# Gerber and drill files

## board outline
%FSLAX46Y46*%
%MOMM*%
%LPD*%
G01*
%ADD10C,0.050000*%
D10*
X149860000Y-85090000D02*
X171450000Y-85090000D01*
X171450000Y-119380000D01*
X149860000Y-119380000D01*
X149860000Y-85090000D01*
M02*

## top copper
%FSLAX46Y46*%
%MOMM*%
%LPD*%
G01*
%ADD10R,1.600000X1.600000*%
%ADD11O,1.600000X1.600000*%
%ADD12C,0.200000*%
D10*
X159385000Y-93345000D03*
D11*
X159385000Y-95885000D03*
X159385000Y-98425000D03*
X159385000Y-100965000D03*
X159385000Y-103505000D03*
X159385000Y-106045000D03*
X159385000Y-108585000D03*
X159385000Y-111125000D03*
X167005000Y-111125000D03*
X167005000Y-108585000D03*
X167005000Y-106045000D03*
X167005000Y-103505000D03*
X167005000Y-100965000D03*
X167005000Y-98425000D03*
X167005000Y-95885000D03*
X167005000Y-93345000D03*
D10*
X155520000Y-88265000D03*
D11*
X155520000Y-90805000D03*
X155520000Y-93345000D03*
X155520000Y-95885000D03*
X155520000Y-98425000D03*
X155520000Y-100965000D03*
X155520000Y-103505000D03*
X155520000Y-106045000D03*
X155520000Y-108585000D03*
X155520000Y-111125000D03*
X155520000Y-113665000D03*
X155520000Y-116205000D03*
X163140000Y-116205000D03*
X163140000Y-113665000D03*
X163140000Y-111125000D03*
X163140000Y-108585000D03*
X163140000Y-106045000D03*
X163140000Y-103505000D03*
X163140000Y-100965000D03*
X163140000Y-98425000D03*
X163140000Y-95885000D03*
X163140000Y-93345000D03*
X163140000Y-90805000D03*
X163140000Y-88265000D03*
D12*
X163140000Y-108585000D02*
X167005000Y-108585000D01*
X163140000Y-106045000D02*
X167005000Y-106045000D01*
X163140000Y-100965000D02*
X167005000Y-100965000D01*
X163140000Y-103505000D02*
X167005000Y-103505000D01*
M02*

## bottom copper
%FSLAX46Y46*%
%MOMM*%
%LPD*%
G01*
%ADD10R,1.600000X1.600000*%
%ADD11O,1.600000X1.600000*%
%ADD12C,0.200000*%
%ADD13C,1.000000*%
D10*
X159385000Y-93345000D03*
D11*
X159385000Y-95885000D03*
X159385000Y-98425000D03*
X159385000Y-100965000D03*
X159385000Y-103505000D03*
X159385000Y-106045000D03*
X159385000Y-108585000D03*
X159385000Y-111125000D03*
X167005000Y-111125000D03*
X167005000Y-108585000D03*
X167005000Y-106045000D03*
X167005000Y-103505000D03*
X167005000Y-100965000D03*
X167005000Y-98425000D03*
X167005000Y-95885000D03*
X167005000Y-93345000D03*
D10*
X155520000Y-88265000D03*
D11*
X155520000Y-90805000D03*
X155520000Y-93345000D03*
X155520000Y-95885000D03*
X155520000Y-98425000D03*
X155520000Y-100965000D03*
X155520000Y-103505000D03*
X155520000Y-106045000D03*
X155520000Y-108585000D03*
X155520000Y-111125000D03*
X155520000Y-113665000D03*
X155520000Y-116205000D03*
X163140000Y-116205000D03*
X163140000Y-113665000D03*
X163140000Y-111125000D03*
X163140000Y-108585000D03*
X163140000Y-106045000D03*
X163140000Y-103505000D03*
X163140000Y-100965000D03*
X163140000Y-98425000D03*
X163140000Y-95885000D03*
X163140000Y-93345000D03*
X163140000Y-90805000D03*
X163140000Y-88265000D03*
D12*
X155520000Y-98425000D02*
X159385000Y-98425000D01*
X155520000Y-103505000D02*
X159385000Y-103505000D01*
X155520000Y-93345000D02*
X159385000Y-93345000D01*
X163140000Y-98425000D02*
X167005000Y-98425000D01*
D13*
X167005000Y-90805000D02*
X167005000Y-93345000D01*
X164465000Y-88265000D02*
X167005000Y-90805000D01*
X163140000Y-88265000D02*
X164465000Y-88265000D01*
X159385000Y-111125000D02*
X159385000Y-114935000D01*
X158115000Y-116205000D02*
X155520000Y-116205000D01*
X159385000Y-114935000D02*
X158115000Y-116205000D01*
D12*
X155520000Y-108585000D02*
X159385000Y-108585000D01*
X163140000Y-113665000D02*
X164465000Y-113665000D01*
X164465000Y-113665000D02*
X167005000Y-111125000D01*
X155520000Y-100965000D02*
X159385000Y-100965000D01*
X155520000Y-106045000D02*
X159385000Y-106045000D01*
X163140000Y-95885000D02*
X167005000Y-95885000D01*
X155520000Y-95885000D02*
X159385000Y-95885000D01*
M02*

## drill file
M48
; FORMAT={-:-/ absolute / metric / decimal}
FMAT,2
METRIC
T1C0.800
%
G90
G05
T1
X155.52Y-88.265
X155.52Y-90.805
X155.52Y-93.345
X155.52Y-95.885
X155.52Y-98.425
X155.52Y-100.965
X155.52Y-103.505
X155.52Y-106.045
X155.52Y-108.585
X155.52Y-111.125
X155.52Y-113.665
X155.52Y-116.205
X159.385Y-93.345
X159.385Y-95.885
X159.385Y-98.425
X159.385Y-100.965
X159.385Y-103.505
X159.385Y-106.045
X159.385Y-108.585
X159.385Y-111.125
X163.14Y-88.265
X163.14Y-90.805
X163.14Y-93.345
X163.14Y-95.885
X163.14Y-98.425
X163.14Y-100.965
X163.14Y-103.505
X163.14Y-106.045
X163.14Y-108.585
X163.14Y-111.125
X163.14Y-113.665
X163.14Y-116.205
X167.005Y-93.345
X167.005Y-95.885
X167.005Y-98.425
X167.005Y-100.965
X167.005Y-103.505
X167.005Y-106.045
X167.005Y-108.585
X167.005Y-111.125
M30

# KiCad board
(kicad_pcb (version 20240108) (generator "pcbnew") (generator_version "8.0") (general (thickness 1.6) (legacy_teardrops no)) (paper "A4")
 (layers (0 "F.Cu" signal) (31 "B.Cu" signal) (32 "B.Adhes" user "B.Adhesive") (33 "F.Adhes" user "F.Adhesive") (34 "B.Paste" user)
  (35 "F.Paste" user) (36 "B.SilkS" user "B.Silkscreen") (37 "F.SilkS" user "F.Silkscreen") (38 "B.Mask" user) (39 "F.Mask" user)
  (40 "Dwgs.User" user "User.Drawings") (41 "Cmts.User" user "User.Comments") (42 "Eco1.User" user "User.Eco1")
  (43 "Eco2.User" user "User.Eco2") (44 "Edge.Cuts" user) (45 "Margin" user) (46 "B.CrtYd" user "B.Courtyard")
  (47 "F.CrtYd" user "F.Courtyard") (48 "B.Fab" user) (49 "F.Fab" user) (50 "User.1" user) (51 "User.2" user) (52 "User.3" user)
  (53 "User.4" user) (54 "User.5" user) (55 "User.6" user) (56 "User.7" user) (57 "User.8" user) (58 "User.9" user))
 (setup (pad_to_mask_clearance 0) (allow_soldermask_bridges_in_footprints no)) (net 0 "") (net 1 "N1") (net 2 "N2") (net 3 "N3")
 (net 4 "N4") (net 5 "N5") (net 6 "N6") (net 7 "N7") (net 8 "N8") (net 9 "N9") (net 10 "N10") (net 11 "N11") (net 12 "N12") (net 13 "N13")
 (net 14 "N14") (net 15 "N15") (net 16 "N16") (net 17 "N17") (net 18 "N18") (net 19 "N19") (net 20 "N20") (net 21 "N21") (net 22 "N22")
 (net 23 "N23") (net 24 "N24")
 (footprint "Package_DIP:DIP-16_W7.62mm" (layer "F.Cu") (at 159.385 93.345)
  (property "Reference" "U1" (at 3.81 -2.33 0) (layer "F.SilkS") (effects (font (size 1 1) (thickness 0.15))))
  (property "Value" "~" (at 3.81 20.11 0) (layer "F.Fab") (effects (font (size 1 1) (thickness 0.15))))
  (pad "1" thru_hole rect (at 0 0) (size 1.6 1.6) (drill 0.8) (layers "*.Cu" "*.Mask") (remove_unused_layers no) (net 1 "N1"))
  (pad "2" thru_hole oval (at 0 2.54) (size 1.6 1.6) (drill 0.8) (layers "*.Cu" "*.Mask") (remove_unused_layers no) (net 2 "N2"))
  (pad "3" thru_hole oval (at 0 5.08) (size 1.6 1.6) (drill 0.8) (layers "*.Cu" "*.Mask") (remove_unused_layers no) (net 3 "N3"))
  (pad "4" thru_hole oval (at 0 7.62) (size 1.6 1.6) (drill 0.8) (layers "*.Cu" "*.Mask") (remove_unused_layers no) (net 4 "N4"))
  (pad "5" thru_hole oval (at 0 10.16) (size 1.6 1.6) (drill 0.8) (layers "*.Cu" "*.Mask") (remove_unused_layers no) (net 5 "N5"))
  (pad "6" thru_hole oval (at 0 12.7) (size 1.6 1.6) (drill 0.8) (layers "*.Cu" "*.Mask") (remove_unused_layers no) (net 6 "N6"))
  (pad "7" thru_hole oval (at 0 15.24) (size 1.6 1.6) (drill 0.8) (layers "*.Cu" "*.Mask") (remove_unused_layers no) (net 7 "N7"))
  (pad "8" thru_hole oval (at 0 17.78) (size 1.6 1.6) (drill 0.8) (layers "*.Cu" "*.Mask") (remove_unused_layers no) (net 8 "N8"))
  (pad "9" thru_hole oval (at 7.62 17.78) (size 1.6 1.6) (drill 0.8) (layers "*.Cu" "*.Mask") (remove_unused_layers no) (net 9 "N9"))
  (pad "10" thru_hole oval (at 7.62 15.24) (size 1.6 1.6) (drill 0.8) (layers "*.Cu" "*.Mask") (remove_unused_layers no) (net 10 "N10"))
  (pad "11" thru_hole oval (at 7.62 12.7) (size 1.6 1.6) (drill 0.8) (layers "*.Cu" "*.Mask") (remove_unused_layers no) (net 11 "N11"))
  (pad "12" thru_hole oval (at 7.62 10.16) (size 1.6 1.6) (drill 0.8) (layers "*.Cu" "*.Mask") (remove_unused_layers no) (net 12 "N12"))
  (pad "13" thru_hole oval (at 7.62 7.62) (size 1.6 1.6) (drill 0.8) (layers "*.Cu" "*.Mask") (remove_unused_layers no) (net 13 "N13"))
  (pad "14" thru_hole oval (at 7.62 5.08) (size 1.6 1.6) (drill 0.8) (layers "*.Cu" "*.Mask") (remove_unused_layers no) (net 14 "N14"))
  (pad "15" thru_hole oval (at 7.62 2.54) (size 1.6 1.6) (drill 0.8) (layers "*.Cu" "*.Mask") (remove_unused_layers no) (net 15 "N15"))
  (pad "16" thru_hole oval (at 7.62 0) (size 1.6 1.6) (drill 0.8) (layers "*.Cu" "*.Mask") (remove_unused_layers no) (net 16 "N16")))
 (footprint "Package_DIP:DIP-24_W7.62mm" (layer "F.Cu") (at 155.52 88.265)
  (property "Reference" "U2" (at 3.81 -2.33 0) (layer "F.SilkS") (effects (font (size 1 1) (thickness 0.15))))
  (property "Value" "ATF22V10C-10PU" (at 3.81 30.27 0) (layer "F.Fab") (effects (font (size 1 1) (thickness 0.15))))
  (pad "1" thru_hole rect (at 0 0) (size 1.6 1.6) (drill 0.8) (layers "*.Cu" "*.Mask") (remove_unused_layers no) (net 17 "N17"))
  (pad "2" thru_hole oval (at 0 2.54) (size 1.6 1.6) (drill 0.8) (layers "*.Cu" "*.Mask") (remove_unused_layers no) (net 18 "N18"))
  (pad "3" thru_hole oval (at 0 5.08) (size 1.6 1.6) (drill 0.8) (layers "*.Cu" "*.Mask") (remove_unused_layers no) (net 1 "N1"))
  (pad "4" thru_hole oval (at 0 7.62) (size 1.6 1.6) (drill 0.8) (layers "*.Cu" "*.Mask") (remove_unused_layers no) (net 2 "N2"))
  (pad "5" thru_hole oval (at 0 10.16) (size 1.6 1.6) (drill 0.8) (layers "*.Cu" "*.Mask") (remove_unused_layers no) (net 3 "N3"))
  (pad "6" thru_hole oval (at 0 12.7) (size 1.6 1.6) (drill 0.8) (layers "*.Cu" "*.Mask") (remove_unused_layers no) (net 4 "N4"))
  (pad "7" thru_hole oval (at 0 15.24) (size 1.6 1.6) (drill 0.8) (layers "*.Cu" "*.Mask") (remove_unused_layers no) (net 5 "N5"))
  (pad "8" thru_hole oval (at 0 17.78) (size 1.6 1.6) (drill 0.8) (layers "*.Cu" "*.Mask") (remove_unused_layers no) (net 6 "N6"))
  (pad "9" thru_hole oval (at 0 20.32) (size 1.6 1.6) (drill 0.8) (layers "*.Cu" "*.Mask") (remove_unused_layers no) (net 7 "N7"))
  (pad "10" thru_hole oval (at 0 22.86) (size 1.6 1.6) (drill 0.8) (layers "*.Cu" "*.Mask") (remove_unused_layers no) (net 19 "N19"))
  (pad "11" thru_hole oval (at 0 25.4) (size 1.6 1.6) (drill 0.8) (layers "*.Cu" "*.Mask") (remove_unused_layers no) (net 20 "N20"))
  (pad "12" thru_hole oval (at 0 27.94) (size 1.6 1.6) (drill 0.8) (layers "*.Cu" "*.Mask") (remove_unused_layers no) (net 8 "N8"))
  (pad "13" thru_hole oval (at 7.62 27.94) (size 1.6 1.6) (drill 0.8) (layers "*.Cu" "*.Mask") (remove_unused_layers no) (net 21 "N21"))
  (pad "14" thru_hole oval (at 7.62 25.4) (size 1.6 1.6) (drill 0.8) (layers "*.Cu" "*.Mask") (remove_unused_layers no) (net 9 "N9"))
  (pad "15" thru_hole oval (at 7.62 22.86) (size 1.6 1.6) (drill 0.8) (layers "*.Cu" "*.Mask") (remove_unused_layers no) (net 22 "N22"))
  (pad "16" thru_hole oval (at 7.62 20.32) (size 1.6 1.6) (drill 0.8) (layers "*.Cu" "*.Mask") (remove_unused_layers no) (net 10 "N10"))
  (pad "17" thru_hole oval (at 7.62 17.78) (size 1.6 1.6) (drill 0.8) (layers "*.Cu" "*.Mask") (remove_unused_layers no) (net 11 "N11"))
  (pad "18" thru_hole oval (at 7.62 15.24) (size 1.6 1.6) (drill 0.8) (layers "*.Cu" "*.Mask") (remove_unused_layers no) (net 12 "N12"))
  (pad "19" thru_hole oval (at 7.62 12.7) (size 1.6 1.6) (drill 0.8) (layers "*.Cu" "*.Mask") (remove_unused_layers no) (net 13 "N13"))
  (pad "20" thru_hole oval (at 7.62 10.16) (size 1.6 1.6) (drill 0.8) (layers "*.Cu" "*.Mask") (remove_unused_layers no) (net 14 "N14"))
  (pad "21" thru_hole oval (at 7.62 7.62) (size 1.6 1.6) (drill 0.8) (layers "*.Cu" "*.Mask") (remove_unused_layers no) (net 15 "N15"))
  (pad "22" thru_hole oval (at 7.62 5.08) (size 1.6 1.6) (drill 0.8) (layers "*.Cu" "*.Mask") (remove_unused_layers no) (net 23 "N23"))
  (pad "23" thru_hole oval (at 7.62 2.54) (size 1.6 1.6) (drill 0.8) (layers "*.Cu" "*.Mask") (remove_unused_layers no) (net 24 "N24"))
  (pad "24" thru_hole oval (at 7.62 0) (size 1.6 1.6) (drill 0.8) (layers "*.Cu" "*.Mask") (remove_unused_layers no) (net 16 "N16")))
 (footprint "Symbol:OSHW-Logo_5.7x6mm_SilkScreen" (layer "F.Cu") (at 167.64 115.57 90)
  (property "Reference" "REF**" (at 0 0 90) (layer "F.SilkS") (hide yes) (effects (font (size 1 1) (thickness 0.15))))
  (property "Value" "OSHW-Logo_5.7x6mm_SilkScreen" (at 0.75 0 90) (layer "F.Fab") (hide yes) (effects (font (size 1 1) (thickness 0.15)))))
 (gr_rect (start 149.86 85.09) (end 171.45 119.38) (stroke (width 0.05) (type default)) (fill none) (layer "Edge.Cuts"))
 (segment (start 155.52 98.425) (end 159.385 98.425) (width 0.2) (layer "B.Cu") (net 3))
 (segment (start 155.52 103.505) (end 159.385 103.505) (width 0.2) (layer "B.Cu") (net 5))
 (segment (start 155.52 93.345) (end 159.385 93.345) (width 0.2) (layer "B.Cu") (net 1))
 (segment (start 163.14 108.585) (end 167.005 108.585) (width 0.2) (layer "F.Cu") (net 10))
 (segment (start 163.14 98.425) (end 167.005 98.425) (width 0.2) (layer "B.Cu") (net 14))
 (segment (start 167.005 90.805) (end 167.005 93.345) (width 1) (layer "B.Cu") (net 16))
 (segment (start 164.465 88.265) (end 167.005 90.805) (width 1) (layer "B.Cu") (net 16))
 (segment (start 163.14 88.265) (end 164.465 88.265) (width 1) (layer "B.Cu") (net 16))
 (segment (start 163.14 106.045) (end 167.005 106.045) (width 0.2) (layer "F.Cu") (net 11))
 (segment (start 159.385 111.125) (end 159.385 114.935) (width 1) (layer "B.Cu") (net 8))
 (segment (start 158.115 116.205) (end 155.52 116.205) (width 1) (layer "B.Cu") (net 8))
 (segment (start 159.385 114.935) (end 158.115 116.205) (width 1) (layer "B.Cu") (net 8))
 (segment (start 163.14 100.965) (end 167.005 100.965) (width 0.2) (layer "F.Cu") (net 13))
 (segment (start 155.52 108.585) (end 159.385 108.585) (width 0.2) (layer "B.Cu") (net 7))
 (segment (start 163.14 113.665) (end 164.465 113.665) (width 0.2) (layer "B.Cu") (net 9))
 (segment (start 164.465 113.665) (end 167.005 111.125) (width 0.2) (layer "B.Cu") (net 9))
 (segment (start 155.52 100.965) (end 159.385 100.965) (width 0.2) (layer "B.Cu") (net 4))
 (segment (start 155.52 106.045) (end 159.385 106.045) (width 0.2) (layer "B.Cu") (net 6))
 (segment (start 163.14 95.885) (end 167.005 95.885) (width 0.2) (layer "B.Cu") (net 15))
 (segment (start 163.14 103.505) (end 167.005 103.505) (width 0.2) (layer "F.Cu") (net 12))
 (segment (start 155.52 95.885) (end 159.385 95.885) (width 0.2) (layer "B.Cu") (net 2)))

